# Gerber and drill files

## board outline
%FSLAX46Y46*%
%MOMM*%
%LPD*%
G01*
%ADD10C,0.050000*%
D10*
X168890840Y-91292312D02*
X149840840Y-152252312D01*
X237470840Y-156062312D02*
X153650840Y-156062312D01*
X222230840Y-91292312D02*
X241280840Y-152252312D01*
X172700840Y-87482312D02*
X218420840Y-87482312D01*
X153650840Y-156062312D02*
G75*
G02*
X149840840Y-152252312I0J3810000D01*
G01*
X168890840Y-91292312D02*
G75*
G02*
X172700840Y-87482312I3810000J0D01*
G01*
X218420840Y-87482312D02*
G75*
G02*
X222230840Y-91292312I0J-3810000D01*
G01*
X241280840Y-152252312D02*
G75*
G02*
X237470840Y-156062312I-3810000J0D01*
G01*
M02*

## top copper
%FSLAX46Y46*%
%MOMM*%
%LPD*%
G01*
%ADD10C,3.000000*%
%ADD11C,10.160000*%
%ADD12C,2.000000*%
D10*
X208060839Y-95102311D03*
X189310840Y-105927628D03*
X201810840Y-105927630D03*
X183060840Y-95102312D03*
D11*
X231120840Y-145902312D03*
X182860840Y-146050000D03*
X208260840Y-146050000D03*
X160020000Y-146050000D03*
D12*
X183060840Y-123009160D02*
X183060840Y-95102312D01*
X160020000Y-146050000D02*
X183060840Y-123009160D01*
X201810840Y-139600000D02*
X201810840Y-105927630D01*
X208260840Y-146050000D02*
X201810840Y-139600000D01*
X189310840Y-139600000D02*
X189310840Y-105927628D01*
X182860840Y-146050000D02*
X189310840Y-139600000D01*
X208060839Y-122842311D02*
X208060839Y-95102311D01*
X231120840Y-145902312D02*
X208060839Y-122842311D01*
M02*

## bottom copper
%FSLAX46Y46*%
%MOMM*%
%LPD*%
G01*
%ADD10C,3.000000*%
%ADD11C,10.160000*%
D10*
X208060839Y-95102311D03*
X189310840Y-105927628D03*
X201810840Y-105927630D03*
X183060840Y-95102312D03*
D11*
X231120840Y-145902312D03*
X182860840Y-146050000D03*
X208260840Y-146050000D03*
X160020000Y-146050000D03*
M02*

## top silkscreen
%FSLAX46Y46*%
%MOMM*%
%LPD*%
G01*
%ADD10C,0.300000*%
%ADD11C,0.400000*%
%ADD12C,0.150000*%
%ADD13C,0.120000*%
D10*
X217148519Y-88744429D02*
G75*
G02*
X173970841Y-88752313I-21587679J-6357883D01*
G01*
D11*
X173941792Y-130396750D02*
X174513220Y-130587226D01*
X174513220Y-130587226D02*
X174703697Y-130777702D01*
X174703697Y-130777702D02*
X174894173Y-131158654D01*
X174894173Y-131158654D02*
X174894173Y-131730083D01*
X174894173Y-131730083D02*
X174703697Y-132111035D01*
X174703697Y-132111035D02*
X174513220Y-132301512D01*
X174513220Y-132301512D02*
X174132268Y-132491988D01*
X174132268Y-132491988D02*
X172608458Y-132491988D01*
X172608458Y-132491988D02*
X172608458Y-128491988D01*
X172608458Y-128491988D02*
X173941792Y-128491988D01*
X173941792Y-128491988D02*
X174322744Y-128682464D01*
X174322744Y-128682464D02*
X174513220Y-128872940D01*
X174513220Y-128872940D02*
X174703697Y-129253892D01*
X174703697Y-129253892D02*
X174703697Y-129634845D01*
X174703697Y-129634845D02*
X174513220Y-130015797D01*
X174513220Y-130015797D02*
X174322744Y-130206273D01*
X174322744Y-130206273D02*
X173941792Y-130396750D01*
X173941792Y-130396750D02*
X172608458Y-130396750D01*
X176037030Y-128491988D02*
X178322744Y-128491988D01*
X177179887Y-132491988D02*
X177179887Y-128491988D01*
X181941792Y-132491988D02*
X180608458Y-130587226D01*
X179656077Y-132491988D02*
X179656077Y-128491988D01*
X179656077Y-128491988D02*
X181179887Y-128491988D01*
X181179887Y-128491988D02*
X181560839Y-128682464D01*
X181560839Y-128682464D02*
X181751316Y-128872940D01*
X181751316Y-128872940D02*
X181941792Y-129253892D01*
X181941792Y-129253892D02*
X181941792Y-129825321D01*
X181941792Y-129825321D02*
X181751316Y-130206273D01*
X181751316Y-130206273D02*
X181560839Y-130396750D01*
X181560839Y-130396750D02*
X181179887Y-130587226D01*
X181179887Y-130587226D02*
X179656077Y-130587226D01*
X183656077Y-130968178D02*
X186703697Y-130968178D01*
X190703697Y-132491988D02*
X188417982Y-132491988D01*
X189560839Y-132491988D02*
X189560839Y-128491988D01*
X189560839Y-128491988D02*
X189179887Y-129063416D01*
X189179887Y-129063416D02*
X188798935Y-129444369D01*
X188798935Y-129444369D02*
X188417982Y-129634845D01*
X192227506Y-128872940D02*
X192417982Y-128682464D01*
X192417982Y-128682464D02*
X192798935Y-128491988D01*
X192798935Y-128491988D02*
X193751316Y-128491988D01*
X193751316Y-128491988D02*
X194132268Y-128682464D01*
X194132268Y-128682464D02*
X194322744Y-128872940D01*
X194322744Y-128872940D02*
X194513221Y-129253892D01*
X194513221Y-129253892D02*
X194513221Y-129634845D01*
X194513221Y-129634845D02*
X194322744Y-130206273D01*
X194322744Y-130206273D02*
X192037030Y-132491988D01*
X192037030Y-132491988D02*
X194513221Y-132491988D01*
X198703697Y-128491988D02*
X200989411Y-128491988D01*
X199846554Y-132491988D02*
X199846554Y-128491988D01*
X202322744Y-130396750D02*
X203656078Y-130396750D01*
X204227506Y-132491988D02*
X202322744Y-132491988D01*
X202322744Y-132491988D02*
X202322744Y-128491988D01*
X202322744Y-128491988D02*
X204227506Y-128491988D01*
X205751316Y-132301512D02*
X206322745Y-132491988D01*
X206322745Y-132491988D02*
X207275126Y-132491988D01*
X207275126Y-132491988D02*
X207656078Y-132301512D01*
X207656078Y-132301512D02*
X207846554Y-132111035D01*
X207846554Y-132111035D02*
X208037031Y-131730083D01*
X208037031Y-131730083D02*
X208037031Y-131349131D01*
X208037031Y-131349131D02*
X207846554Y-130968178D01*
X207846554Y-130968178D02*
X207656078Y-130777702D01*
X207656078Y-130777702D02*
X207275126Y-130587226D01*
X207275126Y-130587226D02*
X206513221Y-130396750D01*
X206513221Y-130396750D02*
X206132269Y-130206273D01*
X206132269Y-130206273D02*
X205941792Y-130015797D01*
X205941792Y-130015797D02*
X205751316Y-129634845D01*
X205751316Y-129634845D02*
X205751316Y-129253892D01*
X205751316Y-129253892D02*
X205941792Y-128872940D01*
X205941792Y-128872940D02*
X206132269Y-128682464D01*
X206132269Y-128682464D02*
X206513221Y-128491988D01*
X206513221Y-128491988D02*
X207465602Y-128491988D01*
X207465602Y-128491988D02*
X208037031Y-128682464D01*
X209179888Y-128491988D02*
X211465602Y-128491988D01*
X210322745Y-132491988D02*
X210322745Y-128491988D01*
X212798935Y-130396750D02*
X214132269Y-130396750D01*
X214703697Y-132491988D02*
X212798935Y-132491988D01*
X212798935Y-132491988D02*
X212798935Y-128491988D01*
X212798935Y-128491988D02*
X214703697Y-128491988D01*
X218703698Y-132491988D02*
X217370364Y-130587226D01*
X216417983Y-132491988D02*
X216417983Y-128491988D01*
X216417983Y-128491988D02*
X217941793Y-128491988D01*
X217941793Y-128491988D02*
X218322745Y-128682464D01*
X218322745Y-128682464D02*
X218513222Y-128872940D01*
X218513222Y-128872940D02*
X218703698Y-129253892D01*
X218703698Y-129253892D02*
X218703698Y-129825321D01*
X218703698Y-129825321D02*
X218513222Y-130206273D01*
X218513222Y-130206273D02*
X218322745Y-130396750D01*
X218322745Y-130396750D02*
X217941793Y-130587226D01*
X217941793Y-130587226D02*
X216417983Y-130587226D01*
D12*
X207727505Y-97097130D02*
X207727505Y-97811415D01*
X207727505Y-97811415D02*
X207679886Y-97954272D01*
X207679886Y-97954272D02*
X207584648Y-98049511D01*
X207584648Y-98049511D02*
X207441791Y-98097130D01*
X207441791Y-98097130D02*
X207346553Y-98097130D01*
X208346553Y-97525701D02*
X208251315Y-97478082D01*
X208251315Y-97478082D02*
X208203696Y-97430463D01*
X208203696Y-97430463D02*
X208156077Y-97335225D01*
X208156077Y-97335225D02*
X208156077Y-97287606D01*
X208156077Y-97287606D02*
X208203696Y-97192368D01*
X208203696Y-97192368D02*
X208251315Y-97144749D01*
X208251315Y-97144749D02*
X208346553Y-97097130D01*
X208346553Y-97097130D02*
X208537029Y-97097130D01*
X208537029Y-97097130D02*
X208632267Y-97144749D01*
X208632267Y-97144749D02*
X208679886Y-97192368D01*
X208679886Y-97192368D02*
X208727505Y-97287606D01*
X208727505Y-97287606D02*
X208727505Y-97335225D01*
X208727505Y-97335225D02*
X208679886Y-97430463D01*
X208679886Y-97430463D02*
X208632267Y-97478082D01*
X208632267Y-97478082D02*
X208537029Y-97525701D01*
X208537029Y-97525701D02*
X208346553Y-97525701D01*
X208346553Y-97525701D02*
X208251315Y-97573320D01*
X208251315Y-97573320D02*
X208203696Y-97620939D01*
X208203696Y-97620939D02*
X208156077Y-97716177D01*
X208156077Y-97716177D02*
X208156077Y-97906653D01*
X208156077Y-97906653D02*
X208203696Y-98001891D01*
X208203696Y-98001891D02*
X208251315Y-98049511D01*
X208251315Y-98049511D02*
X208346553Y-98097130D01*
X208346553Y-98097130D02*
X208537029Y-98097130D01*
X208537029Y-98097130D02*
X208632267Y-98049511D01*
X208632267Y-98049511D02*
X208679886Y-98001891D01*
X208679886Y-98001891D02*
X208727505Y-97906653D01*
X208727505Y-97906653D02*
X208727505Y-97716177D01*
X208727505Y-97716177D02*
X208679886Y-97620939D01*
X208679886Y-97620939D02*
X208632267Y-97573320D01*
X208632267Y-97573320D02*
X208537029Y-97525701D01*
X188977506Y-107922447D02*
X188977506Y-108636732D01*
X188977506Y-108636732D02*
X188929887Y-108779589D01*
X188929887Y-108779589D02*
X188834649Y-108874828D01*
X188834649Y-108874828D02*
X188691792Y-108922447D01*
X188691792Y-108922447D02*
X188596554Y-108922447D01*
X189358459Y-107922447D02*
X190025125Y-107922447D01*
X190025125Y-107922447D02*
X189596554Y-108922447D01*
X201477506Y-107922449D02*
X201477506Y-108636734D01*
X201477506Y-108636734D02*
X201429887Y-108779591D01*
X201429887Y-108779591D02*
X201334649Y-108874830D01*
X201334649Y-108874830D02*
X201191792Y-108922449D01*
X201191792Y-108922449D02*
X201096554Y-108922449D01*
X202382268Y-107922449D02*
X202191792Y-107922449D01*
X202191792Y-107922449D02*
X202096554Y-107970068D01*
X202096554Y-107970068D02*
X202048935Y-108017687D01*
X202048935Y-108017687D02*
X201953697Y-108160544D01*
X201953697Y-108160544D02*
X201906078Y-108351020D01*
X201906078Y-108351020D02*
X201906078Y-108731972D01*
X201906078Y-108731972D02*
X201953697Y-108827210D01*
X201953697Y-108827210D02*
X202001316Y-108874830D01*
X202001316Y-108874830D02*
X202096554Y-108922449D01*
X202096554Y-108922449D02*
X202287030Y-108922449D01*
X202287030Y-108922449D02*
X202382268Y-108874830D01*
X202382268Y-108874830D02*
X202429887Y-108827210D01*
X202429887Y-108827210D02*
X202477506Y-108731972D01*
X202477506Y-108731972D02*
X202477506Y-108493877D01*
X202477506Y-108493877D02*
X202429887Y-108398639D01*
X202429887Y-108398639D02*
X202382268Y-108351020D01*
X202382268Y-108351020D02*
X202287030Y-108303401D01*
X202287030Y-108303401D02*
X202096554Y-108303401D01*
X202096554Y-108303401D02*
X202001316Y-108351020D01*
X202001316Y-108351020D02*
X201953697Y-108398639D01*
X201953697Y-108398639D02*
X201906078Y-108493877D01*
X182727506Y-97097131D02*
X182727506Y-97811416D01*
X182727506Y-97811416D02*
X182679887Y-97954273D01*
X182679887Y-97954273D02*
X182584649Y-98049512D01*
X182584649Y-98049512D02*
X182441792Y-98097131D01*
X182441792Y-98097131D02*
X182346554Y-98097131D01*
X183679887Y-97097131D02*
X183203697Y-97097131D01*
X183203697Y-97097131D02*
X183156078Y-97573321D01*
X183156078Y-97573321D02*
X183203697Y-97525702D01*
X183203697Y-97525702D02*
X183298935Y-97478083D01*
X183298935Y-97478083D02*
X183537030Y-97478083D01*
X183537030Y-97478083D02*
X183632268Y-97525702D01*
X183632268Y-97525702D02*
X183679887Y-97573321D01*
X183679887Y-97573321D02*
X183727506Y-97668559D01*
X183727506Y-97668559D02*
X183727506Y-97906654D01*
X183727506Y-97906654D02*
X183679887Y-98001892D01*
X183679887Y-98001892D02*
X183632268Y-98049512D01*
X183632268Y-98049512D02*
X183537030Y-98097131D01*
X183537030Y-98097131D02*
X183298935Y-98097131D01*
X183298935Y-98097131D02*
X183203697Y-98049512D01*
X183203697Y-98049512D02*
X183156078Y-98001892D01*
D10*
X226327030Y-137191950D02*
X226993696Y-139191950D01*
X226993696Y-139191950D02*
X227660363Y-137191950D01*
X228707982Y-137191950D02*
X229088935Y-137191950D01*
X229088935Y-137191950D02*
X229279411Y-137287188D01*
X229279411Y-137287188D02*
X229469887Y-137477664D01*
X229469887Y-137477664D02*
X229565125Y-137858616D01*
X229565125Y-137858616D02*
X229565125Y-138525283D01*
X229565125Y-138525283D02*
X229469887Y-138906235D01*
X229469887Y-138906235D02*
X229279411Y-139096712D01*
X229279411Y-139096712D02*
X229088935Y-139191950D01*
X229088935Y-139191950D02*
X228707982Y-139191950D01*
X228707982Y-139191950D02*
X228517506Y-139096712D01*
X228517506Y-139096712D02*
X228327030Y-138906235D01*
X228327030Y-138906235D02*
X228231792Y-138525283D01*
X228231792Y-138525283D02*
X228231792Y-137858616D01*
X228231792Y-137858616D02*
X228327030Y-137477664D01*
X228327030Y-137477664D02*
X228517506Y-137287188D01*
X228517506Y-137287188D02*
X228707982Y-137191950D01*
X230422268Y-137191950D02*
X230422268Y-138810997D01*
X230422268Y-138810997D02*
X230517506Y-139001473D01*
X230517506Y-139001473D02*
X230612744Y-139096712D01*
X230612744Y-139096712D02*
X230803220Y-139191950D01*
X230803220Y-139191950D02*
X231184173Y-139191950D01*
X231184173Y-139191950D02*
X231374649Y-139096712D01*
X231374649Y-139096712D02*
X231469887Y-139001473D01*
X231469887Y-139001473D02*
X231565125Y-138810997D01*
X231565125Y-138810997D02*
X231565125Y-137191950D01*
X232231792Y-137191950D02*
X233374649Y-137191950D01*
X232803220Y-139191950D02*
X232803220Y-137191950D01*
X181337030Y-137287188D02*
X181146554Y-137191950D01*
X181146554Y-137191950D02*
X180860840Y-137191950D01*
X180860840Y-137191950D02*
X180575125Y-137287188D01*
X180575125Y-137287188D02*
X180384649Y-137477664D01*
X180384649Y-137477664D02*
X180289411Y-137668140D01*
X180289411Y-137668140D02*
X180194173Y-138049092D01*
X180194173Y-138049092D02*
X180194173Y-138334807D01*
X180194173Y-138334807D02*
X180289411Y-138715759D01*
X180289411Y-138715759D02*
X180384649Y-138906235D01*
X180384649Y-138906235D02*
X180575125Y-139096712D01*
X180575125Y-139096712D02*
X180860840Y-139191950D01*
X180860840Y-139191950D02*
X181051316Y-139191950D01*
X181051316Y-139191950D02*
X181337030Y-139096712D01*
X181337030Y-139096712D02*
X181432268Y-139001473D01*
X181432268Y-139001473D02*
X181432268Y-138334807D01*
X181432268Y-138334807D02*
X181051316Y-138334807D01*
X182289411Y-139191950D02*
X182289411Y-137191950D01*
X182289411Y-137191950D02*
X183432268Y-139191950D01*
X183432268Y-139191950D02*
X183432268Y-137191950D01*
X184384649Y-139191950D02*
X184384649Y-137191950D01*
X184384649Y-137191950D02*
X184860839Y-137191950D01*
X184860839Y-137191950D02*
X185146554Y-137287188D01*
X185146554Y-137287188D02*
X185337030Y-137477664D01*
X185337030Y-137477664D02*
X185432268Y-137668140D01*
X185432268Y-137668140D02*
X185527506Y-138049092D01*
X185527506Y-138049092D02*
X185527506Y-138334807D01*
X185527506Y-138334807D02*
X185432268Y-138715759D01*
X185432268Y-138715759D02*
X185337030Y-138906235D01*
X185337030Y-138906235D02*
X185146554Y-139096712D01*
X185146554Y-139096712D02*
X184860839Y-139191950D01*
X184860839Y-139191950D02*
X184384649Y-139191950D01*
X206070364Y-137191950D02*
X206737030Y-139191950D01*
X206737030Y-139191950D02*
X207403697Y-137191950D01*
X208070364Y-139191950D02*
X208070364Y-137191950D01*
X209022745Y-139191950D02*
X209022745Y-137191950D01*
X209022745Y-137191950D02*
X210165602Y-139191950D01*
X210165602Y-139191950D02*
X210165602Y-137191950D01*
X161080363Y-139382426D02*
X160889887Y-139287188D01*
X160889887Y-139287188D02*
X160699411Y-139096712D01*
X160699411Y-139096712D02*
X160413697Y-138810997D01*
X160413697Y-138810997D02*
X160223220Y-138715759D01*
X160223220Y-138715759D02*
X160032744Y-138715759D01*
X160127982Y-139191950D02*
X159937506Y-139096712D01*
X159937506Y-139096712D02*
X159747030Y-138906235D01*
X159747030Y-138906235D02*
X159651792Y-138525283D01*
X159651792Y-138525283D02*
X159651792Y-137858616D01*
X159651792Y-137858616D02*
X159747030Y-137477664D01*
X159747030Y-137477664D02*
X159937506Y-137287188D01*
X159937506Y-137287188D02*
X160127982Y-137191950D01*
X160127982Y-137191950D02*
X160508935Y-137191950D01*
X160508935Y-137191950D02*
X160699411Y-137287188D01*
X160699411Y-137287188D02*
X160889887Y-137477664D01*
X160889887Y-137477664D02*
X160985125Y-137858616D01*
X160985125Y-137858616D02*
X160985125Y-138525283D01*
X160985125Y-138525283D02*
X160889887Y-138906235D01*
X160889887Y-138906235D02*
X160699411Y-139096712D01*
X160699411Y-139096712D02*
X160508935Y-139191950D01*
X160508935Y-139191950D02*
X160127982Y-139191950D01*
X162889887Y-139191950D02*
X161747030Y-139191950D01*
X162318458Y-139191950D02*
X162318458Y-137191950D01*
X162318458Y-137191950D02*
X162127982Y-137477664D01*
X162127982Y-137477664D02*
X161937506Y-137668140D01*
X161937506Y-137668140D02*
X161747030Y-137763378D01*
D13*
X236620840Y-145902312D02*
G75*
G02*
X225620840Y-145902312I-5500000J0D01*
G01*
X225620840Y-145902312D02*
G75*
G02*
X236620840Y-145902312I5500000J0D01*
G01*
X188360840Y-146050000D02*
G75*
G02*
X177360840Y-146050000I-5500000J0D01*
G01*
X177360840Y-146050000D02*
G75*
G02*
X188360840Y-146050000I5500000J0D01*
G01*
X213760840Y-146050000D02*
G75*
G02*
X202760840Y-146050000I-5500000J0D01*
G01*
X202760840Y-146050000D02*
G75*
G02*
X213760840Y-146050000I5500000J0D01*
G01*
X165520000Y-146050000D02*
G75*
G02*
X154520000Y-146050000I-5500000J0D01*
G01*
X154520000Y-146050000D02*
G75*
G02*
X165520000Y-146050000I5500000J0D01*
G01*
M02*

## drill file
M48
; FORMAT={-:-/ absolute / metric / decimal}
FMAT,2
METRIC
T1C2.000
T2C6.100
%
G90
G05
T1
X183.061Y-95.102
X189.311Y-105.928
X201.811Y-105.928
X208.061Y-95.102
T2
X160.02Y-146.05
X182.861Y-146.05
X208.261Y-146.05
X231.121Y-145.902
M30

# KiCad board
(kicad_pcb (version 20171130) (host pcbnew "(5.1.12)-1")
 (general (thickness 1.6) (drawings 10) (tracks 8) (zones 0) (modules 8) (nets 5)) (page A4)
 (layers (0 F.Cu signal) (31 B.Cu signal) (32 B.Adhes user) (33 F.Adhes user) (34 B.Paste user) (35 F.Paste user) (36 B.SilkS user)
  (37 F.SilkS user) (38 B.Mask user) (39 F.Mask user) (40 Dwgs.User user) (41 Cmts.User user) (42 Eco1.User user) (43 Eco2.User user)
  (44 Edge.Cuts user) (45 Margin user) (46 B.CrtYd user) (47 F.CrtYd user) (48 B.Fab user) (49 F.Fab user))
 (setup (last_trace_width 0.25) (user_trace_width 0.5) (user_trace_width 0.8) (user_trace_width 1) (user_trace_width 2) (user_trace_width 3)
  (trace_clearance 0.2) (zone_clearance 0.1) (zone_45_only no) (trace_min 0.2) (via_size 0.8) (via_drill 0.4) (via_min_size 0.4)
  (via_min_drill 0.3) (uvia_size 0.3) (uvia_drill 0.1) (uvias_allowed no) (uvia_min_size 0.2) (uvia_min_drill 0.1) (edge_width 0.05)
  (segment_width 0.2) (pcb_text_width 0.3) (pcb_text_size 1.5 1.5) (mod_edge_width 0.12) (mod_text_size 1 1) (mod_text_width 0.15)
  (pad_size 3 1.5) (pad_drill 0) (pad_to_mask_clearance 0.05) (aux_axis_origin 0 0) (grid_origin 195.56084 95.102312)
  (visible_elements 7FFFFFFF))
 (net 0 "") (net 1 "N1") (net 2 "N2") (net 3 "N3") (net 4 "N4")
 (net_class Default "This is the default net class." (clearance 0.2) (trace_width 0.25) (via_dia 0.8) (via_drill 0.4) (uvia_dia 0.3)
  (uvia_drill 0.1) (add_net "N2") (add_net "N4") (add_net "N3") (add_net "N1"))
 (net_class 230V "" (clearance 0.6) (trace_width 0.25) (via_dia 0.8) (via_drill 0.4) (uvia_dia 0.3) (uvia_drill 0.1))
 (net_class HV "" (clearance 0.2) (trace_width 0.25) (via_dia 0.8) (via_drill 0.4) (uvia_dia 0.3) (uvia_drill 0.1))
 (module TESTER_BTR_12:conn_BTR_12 (layer F.Cu) (at 208.060839 95.102311)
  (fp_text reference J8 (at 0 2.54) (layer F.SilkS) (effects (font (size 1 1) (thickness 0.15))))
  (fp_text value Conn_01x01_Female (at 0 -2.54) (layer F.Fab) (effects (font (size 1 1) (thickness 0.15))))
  (pad 1 thru_hole circle (at 0 0) (size 3 3) (drill 2) (layers *.Cu *.Mask) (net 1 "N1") (die_length 1)))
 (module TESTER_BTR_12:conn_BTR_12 (layer F.Cu) (at 189.31084 105.927628)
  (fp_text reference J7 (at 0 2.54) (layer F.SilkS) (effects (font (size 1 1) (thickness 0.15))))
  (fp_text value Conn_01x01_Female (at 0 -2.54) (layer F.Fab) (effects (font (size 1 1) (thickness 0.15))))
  (pad 1 thru_hole circle (at 0 0) (size 3 3) (drill 2) (layers *.Cu *.Mask) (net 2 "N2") (die_length 1)))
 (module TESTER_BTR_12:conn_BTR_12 (layer F.Cu) (at 201.81084 105.92763)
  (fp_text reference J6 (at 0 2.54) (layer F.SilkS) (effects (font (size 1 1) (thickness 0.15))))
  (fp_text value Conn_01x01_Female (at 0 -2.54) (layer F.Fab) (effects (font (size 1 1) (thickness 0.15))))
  (pad 1 thru_hole circle (at 0 0) (size 3 3) (drill 2) (layers *.Cu *.Mask) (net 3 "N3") (die_length 1)))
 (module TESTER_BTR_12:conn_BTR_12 (layer F.Cu) (at 183.06084 95.102312)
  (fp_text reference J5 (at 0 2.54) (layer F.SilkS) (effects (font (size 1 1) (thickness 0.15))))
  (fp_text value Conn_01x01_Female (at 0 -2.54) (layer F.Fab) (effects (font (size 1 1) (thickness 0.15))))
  (pad 1 thru_hole circle (at 0 0) (size 3 3) (drill 2) (layers *.Cu *.Mask) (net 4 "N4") (die_length 1)))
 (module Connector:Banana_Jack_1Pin (layer F.Cu) (at 231.12084 145.902312)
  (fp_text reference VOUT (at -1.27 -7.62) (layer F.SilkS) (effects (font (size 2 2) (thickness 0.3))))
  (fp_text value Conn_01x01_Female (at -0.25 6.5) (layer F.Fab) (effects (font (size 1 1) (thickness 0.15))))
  (fp_circle (center 0 0) (end 5.5 0) (layer F.SilkS) (width 0.12))
  (pad 1 thru_hole circle (at 0 0) (size 10.16 10.16) (drill 6.1) (layers *.Cu *.Mask) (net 1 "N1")))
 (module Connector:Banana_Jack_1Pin (layer F.Cu) (at 182.86084 146.05)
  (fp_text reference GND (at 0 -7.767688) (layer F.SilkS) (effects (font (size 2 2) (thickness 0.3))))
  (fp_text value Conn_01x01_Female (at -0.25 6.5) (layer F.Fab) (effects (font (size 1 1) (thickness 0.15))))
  (fp_circle (center 0 0) (end 5.5 0) (layer F.SilkS) (width 0.12))
  (pad 1 thru_hole circle (at 0 0) (size 10.16 10.16) (drill 6.1) (layers *.Cu *.Mask) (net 2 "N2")))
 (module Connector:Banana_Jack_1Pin (layer F.Cu) (at 208.26084 146.05)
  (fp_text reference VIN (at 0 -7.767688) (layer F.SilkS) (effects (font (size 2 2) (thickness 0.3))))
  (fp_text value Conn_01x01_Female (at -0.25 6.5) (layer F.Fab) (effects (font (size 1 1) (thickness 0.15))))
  (fp_circle (center 0 0) (end 5.5 0) (layer F.SilkS) (width 0.12))
  (pad 1 thru_hole circle (at 0 0) (size 10.16 10.16) (drill 6.1) (layers *.Cu *.Mask) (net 3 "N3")))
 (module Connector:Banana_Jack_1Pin (layer F.Cu) (at 160.02 146.05)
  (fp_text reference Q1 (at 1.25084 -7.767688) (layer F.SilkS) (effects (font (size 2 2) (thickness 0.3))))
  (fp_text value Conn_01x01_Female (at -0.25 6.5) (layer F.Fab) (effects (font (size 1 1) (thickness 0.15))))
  (fp_circle (center 0 0) (end 5.5 0) (layer F.SilkS) (width 0.12))
  (pad 1 thru_hole circle (at 0 0) (size 10.16 10.16) (drill 6.1) (layers *.Cu *.Mask) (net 4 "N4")))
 (gr_arc (start 195.56084 95.102312) (end 173.970841 88.752313) (angle -212.8) (layer F.SilkS) (width 0.3))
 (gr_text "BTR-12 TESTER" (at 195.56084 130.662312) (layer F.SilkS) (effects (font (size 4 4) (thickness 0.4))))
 (gr_line (start 168.89084 91.292312) (end 149.84084 152.252312) (layer Edge.Cuts) (width 0.05))
 (gr_line (start 237.47084 156.062312) (end 153.65084 156.062312) (layer Edge.Cuts) (width 0.05))
 (gr_line (start 222.23084 91.292312) (end 241.28084 152.252312) (layer Edge.Cuts) (width 0.05))
 (gr_line (start 172.70084 87.482312) (end 218.42084 87.482312) (layer Edge.Cuts) (width 0.05))
 (gr_arc (start 153.65084 152.252312) (end 149.84084 152.252312) (angle -90) (layer Edge.Cuts) (width 0.05))
 (gr_arc (start 172.70084 91.292312) (end 172.70084 87.482312) (angle -90) (layer Edge.Cuts) (width 0.05))
 (gr_arc (start 218.42084 91.292312) (end 222.23084 91.292312) (angle -90) (layer Edge.Cuts) (width 0.05))
 (gr_arc (start 237.47084 152.252312) (end 237.47084 156.062312) (angle -90) (layer Edge.Cuts) (width 0.05))
 (segment (start 183.06084 123.00916) (end 183.06084 95.102312) (width 2) (layer F.Cu) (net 4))
 (segment (start 160.02 146.05) (end 183.06084 123.00916) (width 2) (layer F.Cu) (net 4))
 (segment (start 201.81084 139.6) (end 201.81084 105.92763) (width 2) (layer F.Cu) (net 3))
 (segment (start 208.26084 146.05) (end 201.81084 139.6) (width 2) (layer F.Cu) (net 3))
 (segment (start 189.31084 139.6) (end 189.31084 105.927628) (width 2) (layer F.Cu) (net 2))
 (segment (start 182.86084 146.05) (end 189.31084 139.6) (width 2) (layer F.Cu) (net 2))
 (segment (start 208.060839 122.842311) (end 208.060839 95.102311) (width 2) (layer F.Cu) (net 1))
 (segment (start 231.12084 145.902312) (end 208.060839 122.842311) (width 2) (layer F.Cu) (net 1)))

